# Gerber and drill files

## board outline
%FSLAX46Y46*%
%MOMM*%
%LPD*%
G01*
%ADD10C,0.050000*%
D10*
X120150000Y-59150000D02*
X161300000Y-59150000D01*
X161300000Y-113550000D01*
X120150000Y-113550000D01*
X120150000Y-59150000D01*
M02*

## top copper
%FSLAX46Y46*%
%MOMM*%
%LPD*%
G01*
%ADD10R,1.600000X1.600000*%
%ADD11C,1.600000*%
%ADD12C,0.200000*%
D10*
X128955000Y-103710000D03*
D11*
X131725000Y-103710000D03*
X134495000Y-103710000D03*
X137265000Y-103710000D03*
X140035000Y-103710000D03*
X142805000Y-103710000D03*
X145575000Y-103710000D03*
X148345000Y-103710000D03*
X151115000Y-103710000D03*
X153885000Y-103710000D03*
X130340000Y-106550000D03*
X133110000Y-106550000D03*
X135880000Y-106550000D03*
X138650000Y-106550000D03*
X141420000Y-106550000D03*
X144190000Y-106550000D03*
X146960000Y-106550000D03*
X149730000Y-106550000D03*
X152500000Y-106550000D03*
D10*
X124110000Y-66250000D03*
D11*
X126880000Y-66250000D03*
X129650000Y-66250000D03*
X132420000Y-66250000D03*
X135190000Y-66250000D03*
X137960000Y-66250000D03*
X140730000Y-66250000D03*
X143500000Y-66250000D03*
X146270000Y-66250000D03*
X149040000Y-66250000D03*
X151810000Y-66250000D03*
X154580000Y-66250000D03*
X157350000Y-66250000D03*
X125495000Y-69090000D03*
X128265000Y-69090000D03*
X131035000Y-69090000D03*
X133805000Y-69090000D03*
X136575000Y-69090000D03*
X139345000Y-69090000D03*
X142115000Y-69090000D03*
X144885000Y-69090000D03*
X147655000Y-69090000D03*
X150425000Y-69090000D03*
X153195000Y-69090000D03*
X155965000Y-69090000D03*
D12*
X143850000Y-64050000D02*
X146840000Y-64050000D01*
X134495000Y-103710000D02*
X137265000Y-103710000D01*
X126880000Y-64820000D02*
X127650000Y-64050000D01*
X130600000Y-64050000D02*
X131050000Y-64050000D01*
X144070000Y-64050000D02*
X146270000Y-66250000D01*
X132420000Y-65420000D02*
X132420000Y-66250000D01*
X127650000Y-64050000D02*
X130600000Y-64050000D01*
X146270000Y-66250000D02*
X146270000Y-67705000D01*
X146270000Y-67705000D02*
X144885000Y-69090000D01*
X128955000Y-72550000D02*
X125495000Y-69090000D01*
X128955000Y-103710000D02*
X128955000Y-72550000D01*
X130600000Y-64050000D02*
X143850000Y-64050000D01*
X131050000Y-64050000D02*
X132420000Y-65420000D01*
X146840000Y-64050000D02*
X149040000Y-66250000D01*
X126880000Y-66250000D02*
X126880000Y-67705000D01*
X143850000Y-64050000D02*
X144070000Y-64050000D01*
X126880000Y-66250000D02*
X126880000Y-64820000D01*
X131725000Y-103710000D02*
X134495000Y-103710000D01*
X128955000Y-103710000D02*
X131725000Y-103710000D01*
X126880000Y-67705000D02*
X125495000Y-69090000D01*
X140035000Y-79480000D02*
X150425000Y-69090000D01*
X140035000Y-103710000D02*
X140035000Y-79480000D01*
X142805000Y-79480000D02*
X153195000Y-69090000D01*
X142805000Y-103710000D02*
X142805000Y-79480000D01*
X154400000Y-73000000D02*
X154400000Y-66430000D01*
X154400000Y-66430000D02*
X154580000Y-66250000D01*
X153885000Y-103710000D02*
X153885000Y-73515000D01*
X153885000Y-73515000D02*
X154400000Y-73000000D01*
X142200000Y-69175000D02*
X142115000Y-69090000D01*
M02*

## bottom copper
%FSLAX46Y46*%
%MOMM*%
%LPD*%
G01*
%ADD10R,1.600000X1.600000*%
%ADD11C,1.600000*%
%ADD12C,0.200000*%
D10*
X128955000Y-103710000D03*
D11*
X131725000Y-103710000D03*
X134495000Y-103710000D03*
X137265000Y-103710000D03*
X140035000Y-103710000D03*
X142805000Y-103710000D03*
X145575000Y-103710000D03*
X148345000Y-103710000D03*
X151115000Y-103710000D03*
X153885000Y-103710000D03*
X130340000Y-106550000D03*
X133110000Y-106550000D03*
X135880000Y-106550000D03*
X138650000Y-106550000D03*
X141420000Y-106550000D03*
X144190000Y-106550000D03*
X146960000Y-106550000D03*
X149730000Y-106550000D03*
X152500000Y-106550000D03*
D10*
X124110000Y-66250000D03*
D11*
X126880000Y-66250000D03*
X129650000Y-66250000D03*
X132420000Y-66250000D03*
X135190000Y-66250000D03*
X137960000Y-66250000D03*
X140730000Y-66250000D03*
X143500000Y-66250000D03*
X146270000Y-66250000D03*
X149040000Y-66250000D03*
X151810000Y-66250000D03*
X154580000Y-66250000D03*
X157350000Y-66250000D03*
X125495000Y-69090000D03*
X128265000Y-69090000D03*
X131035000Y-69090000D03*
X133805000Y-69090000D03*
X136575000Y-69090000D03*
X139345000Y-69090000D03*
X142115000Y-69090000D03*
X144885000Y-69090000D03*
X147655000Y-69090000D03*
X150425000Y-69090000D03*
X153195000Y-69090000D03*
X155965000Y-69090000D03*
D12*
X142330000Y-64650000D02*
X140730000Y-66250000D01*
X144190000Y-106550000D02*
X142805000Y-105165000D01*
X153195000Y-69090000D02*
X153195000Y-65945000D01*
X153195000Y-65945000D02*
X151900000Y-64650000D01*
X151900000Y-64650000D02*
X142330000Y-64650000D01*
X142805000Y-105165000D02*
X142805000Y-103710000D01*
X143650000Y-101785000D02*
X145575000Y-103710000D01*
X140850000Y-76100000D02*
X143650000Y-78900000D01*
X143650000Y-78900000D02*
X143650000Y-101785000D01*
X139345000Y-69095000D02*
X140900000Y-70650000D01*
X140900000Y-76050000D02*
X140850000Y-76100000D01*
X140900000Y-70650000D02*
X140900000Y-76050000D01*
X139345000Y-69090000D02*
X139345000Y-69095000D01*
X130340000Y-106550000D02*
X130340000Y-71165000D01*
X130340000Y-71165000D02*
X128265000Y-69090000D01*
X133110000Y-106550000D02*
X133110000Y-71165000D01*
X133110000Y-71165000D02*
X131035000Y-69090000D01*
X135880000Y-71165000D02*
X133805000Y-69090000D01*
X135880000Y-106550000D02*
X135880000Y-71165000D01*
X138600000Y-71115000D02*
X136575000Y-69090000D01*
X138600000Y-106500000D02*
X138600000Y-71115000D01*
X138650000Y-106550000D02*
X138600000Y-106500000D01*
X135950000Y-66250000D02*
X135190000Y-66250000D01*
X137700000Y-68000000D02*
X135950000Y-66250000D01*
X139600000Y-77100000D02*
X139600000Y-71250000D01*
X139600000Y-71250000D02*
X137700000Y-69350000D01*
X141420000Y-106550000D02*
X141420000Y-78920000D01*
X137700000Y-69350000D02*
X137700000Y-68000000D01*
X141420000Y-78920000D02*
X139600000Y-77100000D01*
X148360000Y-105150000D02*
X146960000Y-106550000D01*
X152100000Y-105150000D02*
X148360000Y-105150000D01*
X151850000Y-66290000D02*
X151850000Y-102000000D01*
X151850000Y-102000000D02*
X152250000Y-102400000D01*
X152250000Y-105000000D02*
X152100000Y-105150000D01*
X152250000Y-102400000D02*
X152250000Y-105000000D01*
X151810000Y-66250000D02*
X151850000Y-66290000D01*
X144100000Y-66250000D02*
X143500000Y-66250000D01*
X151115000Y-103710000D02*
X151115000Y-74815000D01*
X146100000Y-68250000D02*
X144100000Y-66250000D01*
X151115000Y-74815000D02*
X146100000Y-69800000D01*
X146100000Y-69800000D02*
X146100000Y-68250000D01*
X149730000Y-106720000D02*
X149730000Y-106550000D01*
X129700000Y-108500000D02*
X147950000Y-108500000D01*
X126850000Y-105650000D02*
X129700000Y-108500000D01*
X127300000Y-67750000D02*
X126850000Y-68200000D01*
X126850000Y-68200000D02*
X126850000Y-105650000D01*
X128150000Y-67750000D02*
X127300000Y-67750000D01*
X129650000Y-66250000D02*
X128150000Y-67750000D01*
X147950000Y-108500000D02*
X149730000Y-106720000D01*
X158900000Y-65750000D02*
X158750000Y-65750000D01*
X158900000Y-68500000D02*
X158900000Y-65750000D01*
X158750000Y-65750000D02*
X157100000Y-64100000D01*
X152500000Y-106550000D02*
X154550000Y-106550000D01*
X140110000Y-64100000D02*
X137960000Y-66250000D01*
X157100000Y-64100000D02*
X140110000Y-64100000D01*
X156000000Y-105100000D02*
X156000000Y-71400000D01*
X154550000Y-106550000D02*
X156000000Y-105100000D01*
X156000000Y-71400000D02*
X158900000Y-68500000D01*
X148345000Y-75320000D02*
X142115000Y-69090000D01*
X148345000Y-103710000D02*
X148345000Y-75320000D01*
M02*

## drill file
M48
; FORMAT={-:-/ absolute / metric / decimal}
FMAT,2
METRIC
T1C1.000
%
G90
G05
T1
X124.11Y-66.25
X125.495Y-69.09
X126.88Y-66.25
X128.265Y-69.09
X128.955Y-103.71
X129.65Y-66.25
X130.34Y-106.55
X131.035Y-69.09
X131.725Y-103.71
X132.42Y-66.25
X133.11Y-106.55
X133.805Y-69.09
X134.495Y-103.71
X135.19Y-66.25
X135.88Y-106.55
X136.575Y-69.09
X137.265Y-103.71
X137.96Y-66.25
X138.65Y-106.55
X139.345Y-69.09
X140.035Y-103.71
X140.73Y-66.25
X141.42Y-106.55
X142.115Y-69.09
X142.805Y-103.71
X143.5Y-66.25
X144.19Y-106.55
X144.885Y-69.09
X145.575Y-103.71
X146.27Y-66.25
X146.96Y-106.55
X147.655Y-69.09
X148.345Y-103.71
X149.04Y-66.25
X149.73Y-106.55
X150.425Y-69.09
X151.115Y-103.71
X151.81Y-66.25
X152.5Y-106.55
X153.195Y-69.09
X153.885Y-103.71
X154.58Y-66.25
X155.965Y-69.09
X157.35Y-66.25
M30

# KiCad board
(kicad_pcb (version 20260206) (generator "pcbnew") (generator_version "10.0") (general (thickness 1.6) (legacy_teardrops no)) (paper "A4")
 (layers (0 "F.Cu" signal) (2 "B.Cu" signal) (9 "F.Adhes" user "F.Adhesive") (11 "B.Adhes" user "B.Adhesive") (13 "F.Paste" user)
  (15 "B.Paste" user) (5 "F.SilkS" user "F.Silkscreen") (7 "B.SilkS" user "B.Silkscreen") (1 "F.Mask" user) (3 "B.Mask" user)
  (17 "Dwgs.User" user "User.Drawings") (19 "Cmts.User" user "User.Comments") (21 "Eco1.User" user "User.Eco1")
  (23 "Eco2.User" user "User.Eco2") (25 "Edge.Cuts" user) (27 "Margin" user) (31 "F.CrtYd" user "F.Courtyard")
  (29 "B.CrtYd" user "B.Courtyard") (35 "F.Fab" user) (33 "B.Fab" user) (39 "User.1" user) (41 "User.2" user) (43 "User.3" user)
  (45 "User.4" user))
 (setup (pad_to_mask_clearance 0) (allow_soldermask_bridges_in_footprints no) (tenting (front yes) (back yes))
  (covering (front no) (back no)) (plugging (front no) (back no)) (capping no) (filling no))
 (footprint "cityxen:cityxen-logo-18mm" (layer "F.Cu") (at 150.123418 88.011446)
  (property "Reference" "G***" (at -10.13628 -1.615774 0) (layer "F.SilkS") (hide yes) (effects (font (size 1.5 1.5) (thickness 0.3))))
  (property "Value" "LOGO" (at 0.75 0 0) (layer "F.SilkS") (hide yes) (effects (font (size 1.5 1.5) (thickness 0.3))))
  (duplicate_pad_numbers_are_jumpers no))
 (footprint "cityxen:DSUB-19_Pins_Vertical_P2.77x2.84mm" (layer "F.Cu") (at 128.955 103.71)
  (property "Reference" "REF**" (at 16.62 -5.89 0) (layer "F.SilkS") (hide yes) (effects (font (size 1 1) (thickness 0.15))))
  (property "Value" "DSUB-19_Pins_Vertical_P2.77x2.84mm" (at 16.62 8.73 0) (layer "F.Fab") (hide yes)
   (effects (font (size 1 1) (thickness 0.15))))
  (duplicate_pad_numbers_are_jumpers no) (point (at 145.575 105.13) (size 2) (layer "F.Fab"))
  (pad "1" thru_hole rect (at 0 0) (size 1.6 1.6) (drill 1) (layers "*.Cu" "*.Mask") (remove_unused_layers no) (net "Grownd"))
  (pad "2" thru_hole circle (at 2.77 0) (size 1.6 1.6) (drill 1) (layers "*.Cu" "*.Mask") (remove_unused_layers no) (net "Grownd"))
  (pad "3" thru_hole circle (at 5.54 0) (size 1.6 1.6) (drill 1) (layers "*.Cu" "*.Mask") (remove_unused_layers no) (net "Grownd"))
  (pad "4" thru_hole circle (at 8.31 0) (size 1.6 1.6) (drill 1) (layers "*.Cu" "*.Mask") (remove_unused_layers no) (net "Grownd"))
  (pad "5" thru_hole circle (at 11.08 0) (size 1.6 1.6) (drill 1) (layers "*.Cu" "*.Mask") (remove_unused_layers no) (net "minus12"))
  (pad "6" thru_hole circle (at 13.85 0) (size 1.6 1.6) (drill 1) (layers "*.Cu" "*.Mask") (remove_unused_layers no) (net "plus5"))
  (pad "7" thru_hole circle (at 16.62 0) (size 1.6 1.6) (drill 1) (layers "*.Cu" "*.Mask") (remove_unused_layers no) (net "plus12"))
  (pad "8" thru_hole circle (at 19.39 0) (size 1.6 1.6) (drill 1) (layers "*.Cu" "*.Mask") (remove_unused_layers no) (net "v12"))
  (pad "9" thru_hole circle (at 22.16 0) (size 1.6 1.6) (drill 1) (layers "*.Cu" "*.Mask") (remove_unused_layers no) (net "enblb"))
  (pad "10" thru_hole circle (at 24.93 0) (size 1.6 1.6) (drill 1) (layers "*.Cu" "*.Mask") (remove_unused_layers no) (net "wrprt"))
  (pad "11" thru_hole circle (at 1.385 2.84) (size 1.6 1.6) (drill 1) (layers "*.Cu" "*.Mask") (remove_unused_layers no) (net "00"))
  (pad "12" thru_hole circle (at 4.155 2.84) (size 1.6 1.6) (drill 1) (layers "*.Cu" "*.Mask") (remove_unused_layers no) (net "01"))
  (pad "13" thru_hole circle (at 6.925 2.84) (size 1.6 1.6) (drill 1) (layers "*.Cu" "*.Mask") (remove_unused_layers no) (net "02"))
  (pad "14" thru_hole circle (at 9.695 2.84) (size 1.6 1.6) (drill 1) (layers "*.Cu" "*.Mask") (remove_unused_layers no) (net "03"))
  (pad "15" thru_hole circle (at 12.465 2.84) (size 1.6 1.6) (drill 1) (layers "*.Cu" "*.Mask") (remove_unused_layers no) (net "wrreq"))
  (pad "16" thru_hole circle (at 15.235 2.84) (size 1.6 1.6) (drill 1) (layers "*.Cu" "*.Mask") (remove_unused_layers no) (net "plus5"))
  (pad "17" thru_hole circle (at 18.005 2.84) (size 1.6 1.6) (drill 1) (layers "*.Cu" "*.Mask") (remove_unused_layers no) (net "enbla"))
  (pad "18" thru_hole circle (at 20.775 2.84) (size 1.6 1.6) (drill 1) (layers "*.Cu" "*.Mask") (remove_unused_layers no) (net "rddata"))
  (pad "19" thru_hole circle (at 23.545 2.84) (size 1.6 1.6) (drill 1) (layers "*.Cu" "*.Mask") (remove_unused_layers no) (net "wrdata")))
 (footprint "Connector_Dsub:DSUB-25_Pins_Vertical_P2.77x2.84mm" (layer "F.Cu") (at 124.11 66.25)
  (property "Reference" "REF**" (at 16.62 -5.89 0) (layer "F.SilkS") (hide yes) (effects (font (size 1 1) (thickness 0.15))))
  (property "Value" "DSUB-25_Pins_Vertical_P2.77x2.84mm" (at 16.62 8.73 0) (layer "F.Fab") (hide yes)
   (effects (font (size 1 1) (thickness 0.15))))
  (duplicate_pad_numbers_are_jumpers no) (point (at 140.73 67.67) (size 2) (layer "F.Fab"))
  (pad "1" thru_hole rect (at 0 0) (size 1.6 1.6) (drill 1) (layers "*.Cu" "*.Mask") (remove_unused_layers no))
  (pad "2" thru_hole circle (at 2.77 0) (size 1.6 1.6) (drill 1) (layers "*.Cu" "*.Mask") (remove_unused_layers no) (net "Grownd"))
  (pad "3" thru_hole circle (at 5.54 0) (size 1.6 1.6) (drill 1) (layers "*.Cu" "*.Mask") (remove_unused_layers no) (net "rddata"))
  (pad "4" thru_hole circle (at 8.31 0) (size 1.6 1.6) (drill 1) (layers "*.Cu" "*.Mask") (remove_unused_layers no) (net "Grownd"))
  (pad "5" thru_hole circle (at 11.08 0) (size 1.6 1.6) (drill 1) (layers "*.Cu" "*.Mask") (remove_unused_layers no) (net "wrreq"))
  (pad "6" thru_hole circle (at 13.85 0) (size 1.6 1.6) (drill 1) (layers "*.Cu" "*.Mask") (remove_unused_layers no) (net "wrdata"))
  (pad "7" thru_hole circle (at 16.62 0) (size 1.6 1.6) (drill 1) (layers "*.Cu" "*.Mask") (remove_unused_layers no) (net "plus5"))
  (pad "8" thru_hole circle (at 19.39 0) (size 1.6 1.6) (drill 1) (layers "*.Cu" "*.Mask") (remove_unused_layers no) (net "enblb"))
  (pad "9" thru_hole circle (at 22.16 0) (size 1.6 1.6) (drill 1) (layers "*.Cu" "*.Mask") (remove_unused_layers no) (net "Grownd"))
  (pad "10" thru_hole circle (at 24.93 0) (size 1.6 1.6) (drill 1) (layers "*.Cu" "*.Mask") (remove_unused_layers no) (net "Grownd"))
  (pad "11" thru_hole circle (at 27.7 0) (size 1.6 1.6) (drill 1) (layers "*.Cu" "*.Mask") (remove_unused_layers no) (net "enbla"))
  (pad "12" thru_hole circle (at 30.47 0) (size 1.6 1.6) (drill 1) (layers "*.Cu" "*.Mask") (remove_unused_layers no) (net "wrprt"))
  (pad "13" thru_hole circle (at 33.24 0) (size 1.6 1.6) (drill 1) (layers "*.Cu" "*.Mask") (remove_unused_layers no))
  (pad "14" thru_hole circle (at 1.385 2.84) (size 1.6 1.6) (drill 1) (layers "*.Cu" "*.Mask") (remove_unused_layers no) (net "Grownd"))
  (pad "15" thru_hole circle (at 4.155 2.84) (size 1.6 1.6) (drill 1) (layers "*.Cu" "*.Mask") (remove_unused_layers no) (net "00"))
  (pad "16" thru_hole circle (at 6.925 2.84) (size 1.6 1.6) (drill 1) (layers "*.Cu" "*.Mask") (remove_unused_layers no) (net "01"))
  (pad "17" thru_hole circle (at 9.695 2.84) (size 1.6 1.6) (drill 1) (layers "*.Cu" "*.Mask") (remove_unused_layers no) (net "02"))
  (pad "18" thru_hole circle (at 12.465 2.84) (size 1.6 1.6) (drill 1) (layers "*.Cu" "*.Mask") (remove_unused_layers no) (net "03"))
  (pad "19" thru_hole circle (at 15.235 2.84) (size 1.6 1.6) (drill 1) (layers "*.Cu" "*.Mask") (remove_unused_layers no) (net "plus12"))
  (pad "20" thru_hole circle (at 18.005 2.84) (size 1.6 1.6) (drill 1) (layers "*.Cu" "*.Mask") (remove_unused_layers no) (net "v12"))
  (pad "21" thru_hole circle (at 20.775 2.84) (size 1.6 1.6) (drill 1) (layers "*.Cu" "*.Mask") (remove_unused_layers no) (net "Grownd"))
  (pad "22" thru_hole circle (at 23.545 2.84) (size 1.6 1.6) (drill 1) (layers "*.Cu" "*.Mask") (remove_unused_layers no))
  (pad "23" thru_hole circle (at 26.315 2.84) (size 1.6 1.6) (drill 1) (layers "*.Cu" "*.Mask") (remove_unused_layers no) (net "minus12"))
  (pad "24" thru_hole circle (at 29.085 2.84) (size 1.6 1.6) (drill 1) (layers "*.Cu" "*.Mask") (remove_unused_layers no) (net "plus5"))
  (pad "25" thru_hole circle (at 31.855 2.84) (size 1.6 1.6) (drill 1) (layers "*.Cu" "*.Mask") (remove_unused_layers no)))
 (gr_rect (start 120.15 59.15) (end 161.3 113.55) (stroke (width 0.05) (type default)) (fill no) (layer "Edge.Cuts"))
 (segment (start 143.85 64.05) (end 146.84 64.05) (width 0.2) (layer "F.Cu") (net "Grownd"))
 (segment (start 134.495 103.71) (end 137.265 103.71) (width 0.2) (layer "F.Cu") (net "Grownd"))
 (segment (start 126.88 64.82) (end 127.65 64.05) (width 0.2) (layer "F.Cu") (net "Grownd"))
 (segment (start 130.6 64.05) (end 131.05 64.05) (width 0.2) (layer "F.Cu") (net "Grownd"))
 (segment (start 144.07 64.05) (end 146.27 66.25) (width 0.2) (layer "F.Cu") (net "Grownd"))
 (segment (start 132.42 65.42) (end 132.42 66.25) (width 0.2) (layer "F.Cu") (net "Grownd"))
 (segment (start 127.65 64.05) (end 130.6 64.05) (width 0.2) (layer "F.Cu") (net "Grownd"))
 (segment (start 146.27 66.25) (end 146.27 67.705) (width 0.2) (layer "F.Cu") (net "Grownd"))
 (segment (start 146.27 67.705) (end 144.885 69.09) (width 0.2) (layer "F.Cu") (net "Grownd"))
 (segment (start 128.955 72.55) (end 125.495 69.09) (width 0.2) (layer "F.Cu") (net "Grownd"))
 (segment (start 128.955 103.71) (end 128.955 72.55) (width 0.2) (layer "F.Cu") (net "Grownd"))
 (segment (start 130.6 64.05) (end 143.85 64.05) (width 0.2) (layer "F.Cu") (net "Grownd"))
 (segment (start 131.05 64.05) (end 132.42 65.42) (width 0.2) (layer "F.Cu") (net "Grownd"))
 (segment (start 146.84 64.05) (end 149.04 66.25) (width 0.2) (layer "F.Cu") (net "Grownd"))
 (segment (start 126.88 66.25) (end 126.88 67.705) (width 0.2) (layer "F.Cu") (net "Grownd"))
 (segment (start 143.85 64.05) (end 144.07 64.05) (width 0.2) (layer "F.Cu") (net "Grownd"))
 (segment (start 126.88 66.25) (end 126.88 64.82) (width 0.2) (layer "F.Cu") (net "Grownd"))
 (segment (start 131.725 103.71) (end 134.495 103.71) (width 0.2) (layer "F.Cu") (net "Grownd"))
 (segment (start 128.955 103.71) (end 131.725 103.71) (width 0.2) (layer "F.Cu") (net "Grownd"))
 (segment (start 126.88 67.705) (end 125.495 69.09) (width 0.2) (layer "F.Cu") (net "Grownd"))
 (segment (start 140.035 79.48) (end 150.425 69.09) (width 0.2) (layer "F.Cu") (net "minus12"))
 (segment (start 140.035 103.71) (end 140.035 79.48) (width 0.2) (layer "F.Cu") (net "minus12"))
 (segment (start 142.805 79.48) (end 153.195 69.09) (width 0.2) (layer "F.Cu") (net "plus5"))
 (segment (start 142.805 103.71) (end 142.805 79.48) (width 0.2) (layer "F.Cu") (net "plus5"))
 (segment (start 142.33 64.65) (end 140.73 66.25) (width 0.2) (layer "B.Cu") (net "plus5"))
 (segment (start 144.19 106.55) (end 142.805 105.165) (width 0.2) (layer "B.Cu") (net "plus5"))
 (segment (start 153.195 69.09) (end 153.195 65.945) (width 0.2) (layer "B.Cu") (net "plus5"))
 (segment (start 153.195 65.945) (end 151.9 64.65) (width 0.2) (layer "B.Cu") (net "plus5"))
 (segment (start 151.9 64.65) (end 142.33 64.65) (width 0.2) (layer "B.Cu") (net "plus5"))
 (segment (start 142.805 105.165) (end 142.805 103.71) (width 0.2) (layer "B.Cu") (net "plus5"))
 (segment (start 143.65 101.785) (end 145.575 103.71) (width 0.2) (layer "B.Cu") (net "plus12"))
 (segment (start 140.85 76.1) (end 143.65 78.9) (width 0.2) (layer "B.Cu") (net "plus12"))
 (segment (start 143.65 78.9) (end 143.65 101.785) (width 0.2) (layer "B.Cu") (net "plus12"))
 (segment (start 139.345 69.095) (end 140.9 70.65) (width 0.2) (layer "B.Cu") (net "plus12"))
 (segment (start 140.9 76.05) (end 140.85 76.1) (width 0.2) (layer "B.Cu") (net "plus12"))
 (segment (start 140.9 70.65) (end 140.9 76.05) (width 0.2) (layer "B.Cu") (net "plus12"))
 (segment (start 139.345 69.09) (end 139.345 69.095) (width 0.2) (layer "B.Cu") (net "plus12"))
 (segment (start 154.4 73) (end 154.4 66.43) (width 0.2) (layer "F.Cu") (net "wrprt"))
 (segment (start 154.4 66.43) (end 154.58 66.25) (width 0.2) (layer "F.Cu") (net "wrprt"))
 (segment (start 153.885 103.71) (end 153.885 73.515) (width 0.2) (layer "F.Cu") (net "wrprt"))
 (segment (start 153.885 73.515) (end 154.4 73) (width 0.2) (layer "F.Cu") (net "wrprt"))
 (segment (start 130.34 106.55) (end 130.34 71.165) (width 0.2) (layer "B.Cu") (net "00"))
 (segment (start 130.34 71.165) (end 128.265 69.09) (width 0.2) (layer "B.Cu") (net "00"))
 (segment (start 133.11 106.55) (end 133.11 71.165) (width 0.2) (layer "B.Cu") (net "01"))
 (segment (start 133.11 71.165) (end 131.035 69.09) (width 0.2) (layer "B.Cu") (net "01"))
 (segment (start 135.88 71.165) (end 133.805 69.09) (width 0.2) (layer "B.Cu") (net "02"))
 (segment (start 135.88 106.55) (end 135.88 71.165) (width 0.2) (layer "B.Cu") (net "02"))
 (segment (start 138.6 71.115) (end 136.575 69.09) (width 0.2) (layer "B.Cu") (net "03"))
 (segment (start 138.6 106.5) (end 138.6 71.115) (width 0.2) (layer "B.Cu") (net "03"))
 (segment (start 138.65 106.55) (end 138.6 106.5) (width 0.2) (layer "B.Cu") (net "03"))
 (segment (start 135.95 66.25) (end 135.19 66.25) (width 0.2) (layer "B.Cu") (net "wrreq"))
 (segment (start 137.7 68) (end 135.95 66.25) (width 0.2) (layer "B.Cu") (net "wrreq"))
 (segment (start 139.6 77.1) (end 139.6 71.25) (width 0.2) (layer "B.Cu") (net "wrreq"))
 (segment (start 139.6 71.25) (end 137.7 69.35) (width 0.2) (layer "B.Cu") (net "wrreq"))
 (segment (start 141.42 106.55) (end 141.42 78.92) (width 0.2) (layer "B.Cu") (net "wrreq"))
 (segment (start 137.7 69.35) (end 137.7 68) (width 0.2) (layer "B.Cu") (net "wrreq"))
 (segment (start 141.42 78.92) (end 139.6 77.1) (width 0.2) (layer "B.Cu") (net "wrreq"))
 (segment (start 148.36 105.15) (end 146.96 106.55) (width 0.2) (layer "B.Cu") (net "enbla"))
 (segment (start 152.1 105.15) (end 148.36 105.15) (width 0.2) (layer "B.Cu") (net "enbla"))
 (segment (start 151.85 66.29) (end 151.85 102) (width 0.2) (layer "B.Cu") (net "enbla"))
 (segment (start 151.85 102) (end 152.25 102.4) (width 0.2) (layer "B.Cu") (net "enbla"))
 (segment (start 152.25 105) (end 152.1 105.15) (width 0.2) (layer "B.Cu") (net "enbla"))
 (segment (start 152.25 102.4) (end 152.25 105) (width 0.2) (layer "B.Cu") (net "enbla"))
 (segment (start 151.81 66.25) (end 151.85 66.29) (width 0.2) (layer "B.Cu") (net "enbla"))
 (segment (start 144.1 66.25) (end 143.5 66.25) (width 0.2) (layer "B.Cu") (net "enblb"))
 (segment (start 151.115 103.71) (end 151.115 74.815) (width 0.2) (layer "B.Cu") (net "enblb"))
 (segment (start 146.1 68.25) (end 144.1 66.25) (width 0.2) (layer "B.Cu") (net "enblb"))
 (segment (start 151.115 74.815) (end 146.1 69.8) (width 0.2) (layer "B.Cu") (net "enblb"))
 (segment (start 146.1 69.8) (end 146.1 68.25) (width 0.2) (layer "B.Cu") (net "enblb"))
 (segment (start 149.73 106.72) (end 149.73 106.55) (width 0.2) (layer "B.Cu") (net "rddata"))
 (segment (start 129.7 108.5) (end 147.95 108.5) (width 0.2) (layer "B.Cu") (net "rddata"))
 (segment (start 126.85 105.65) (end 129.7 108.5) (width 0.2) (layer "B.Cu") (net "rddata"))
 (segment (start 127.3 67.75) (end 126.85 68.2) (width 0.2) (layer "B.Cu") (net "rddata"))
 (segment (start 126.85 68.2) (end 126.85 105.65) (width 0.2) (layer "B.Cu") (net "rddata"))
 (segment (start 128.15 67.75) (end 127.3 67.75) (width 0.2) (layer "B.Cu") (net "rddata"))
 (segment (start 129.65 66.25) (end 128.15 67.75) (width 0.2) (layer "B.Cu") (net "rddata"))
 (segment (start 147.95 108.5) (end 149.73 106.72) (width 0.2) (layer "B.Cu") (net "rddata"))
 (segment (start 158.9 65.75) (end 158.75 65.75) (width 0.2) (layer "B.Cu") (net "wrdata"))
 (segment (start 158.9 68.5) (end 158.9 65.75) (width 0.2) (layer "B.Cu") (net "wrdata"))
 (segment (start 158.75 65.75) (end 157.1 64.1) (width 0.2) (layer "B.Cu") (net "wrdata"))
 (segment (start 152.5 106.55) (end 154.55 106.55) (width 0.2) (layer "B.Cu") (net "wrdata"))
 (segment (start 140.11 64.1) (end 137.96 66.25) (width 0.2) (layer "B.Cu") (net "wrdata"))
 (segment (start 157.1 64.1) (end 140.11 64.1) (width 0.2) (layer "B.Cu") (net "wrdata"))
 (segment (start 156 105.1) (end 156 71.4) (width 0.2) (layer "B.Cu") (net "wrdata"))
 (segment (start 154.55 106.55) (end 156 105.1) (width 0.2) (layer "B.Cu") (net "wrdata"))
 (segment (start 156 71.4) (end 158.9 68.5) (width 0.2) (layer "B.Cu") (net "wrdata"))
 (segment (start 142.2 69.175) (end 142.115 69.09) (width 0.2) (layer "F.Cu") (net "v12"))
 (segment (start 148.345 75.32) (end 142.115 69.09) (width 0.2) (layer "B.Cu") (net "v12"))
 (segment (start 148.345 103.71) (end 148.345 75.32) (width 0.2) (layer "B.Cu") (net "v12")))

